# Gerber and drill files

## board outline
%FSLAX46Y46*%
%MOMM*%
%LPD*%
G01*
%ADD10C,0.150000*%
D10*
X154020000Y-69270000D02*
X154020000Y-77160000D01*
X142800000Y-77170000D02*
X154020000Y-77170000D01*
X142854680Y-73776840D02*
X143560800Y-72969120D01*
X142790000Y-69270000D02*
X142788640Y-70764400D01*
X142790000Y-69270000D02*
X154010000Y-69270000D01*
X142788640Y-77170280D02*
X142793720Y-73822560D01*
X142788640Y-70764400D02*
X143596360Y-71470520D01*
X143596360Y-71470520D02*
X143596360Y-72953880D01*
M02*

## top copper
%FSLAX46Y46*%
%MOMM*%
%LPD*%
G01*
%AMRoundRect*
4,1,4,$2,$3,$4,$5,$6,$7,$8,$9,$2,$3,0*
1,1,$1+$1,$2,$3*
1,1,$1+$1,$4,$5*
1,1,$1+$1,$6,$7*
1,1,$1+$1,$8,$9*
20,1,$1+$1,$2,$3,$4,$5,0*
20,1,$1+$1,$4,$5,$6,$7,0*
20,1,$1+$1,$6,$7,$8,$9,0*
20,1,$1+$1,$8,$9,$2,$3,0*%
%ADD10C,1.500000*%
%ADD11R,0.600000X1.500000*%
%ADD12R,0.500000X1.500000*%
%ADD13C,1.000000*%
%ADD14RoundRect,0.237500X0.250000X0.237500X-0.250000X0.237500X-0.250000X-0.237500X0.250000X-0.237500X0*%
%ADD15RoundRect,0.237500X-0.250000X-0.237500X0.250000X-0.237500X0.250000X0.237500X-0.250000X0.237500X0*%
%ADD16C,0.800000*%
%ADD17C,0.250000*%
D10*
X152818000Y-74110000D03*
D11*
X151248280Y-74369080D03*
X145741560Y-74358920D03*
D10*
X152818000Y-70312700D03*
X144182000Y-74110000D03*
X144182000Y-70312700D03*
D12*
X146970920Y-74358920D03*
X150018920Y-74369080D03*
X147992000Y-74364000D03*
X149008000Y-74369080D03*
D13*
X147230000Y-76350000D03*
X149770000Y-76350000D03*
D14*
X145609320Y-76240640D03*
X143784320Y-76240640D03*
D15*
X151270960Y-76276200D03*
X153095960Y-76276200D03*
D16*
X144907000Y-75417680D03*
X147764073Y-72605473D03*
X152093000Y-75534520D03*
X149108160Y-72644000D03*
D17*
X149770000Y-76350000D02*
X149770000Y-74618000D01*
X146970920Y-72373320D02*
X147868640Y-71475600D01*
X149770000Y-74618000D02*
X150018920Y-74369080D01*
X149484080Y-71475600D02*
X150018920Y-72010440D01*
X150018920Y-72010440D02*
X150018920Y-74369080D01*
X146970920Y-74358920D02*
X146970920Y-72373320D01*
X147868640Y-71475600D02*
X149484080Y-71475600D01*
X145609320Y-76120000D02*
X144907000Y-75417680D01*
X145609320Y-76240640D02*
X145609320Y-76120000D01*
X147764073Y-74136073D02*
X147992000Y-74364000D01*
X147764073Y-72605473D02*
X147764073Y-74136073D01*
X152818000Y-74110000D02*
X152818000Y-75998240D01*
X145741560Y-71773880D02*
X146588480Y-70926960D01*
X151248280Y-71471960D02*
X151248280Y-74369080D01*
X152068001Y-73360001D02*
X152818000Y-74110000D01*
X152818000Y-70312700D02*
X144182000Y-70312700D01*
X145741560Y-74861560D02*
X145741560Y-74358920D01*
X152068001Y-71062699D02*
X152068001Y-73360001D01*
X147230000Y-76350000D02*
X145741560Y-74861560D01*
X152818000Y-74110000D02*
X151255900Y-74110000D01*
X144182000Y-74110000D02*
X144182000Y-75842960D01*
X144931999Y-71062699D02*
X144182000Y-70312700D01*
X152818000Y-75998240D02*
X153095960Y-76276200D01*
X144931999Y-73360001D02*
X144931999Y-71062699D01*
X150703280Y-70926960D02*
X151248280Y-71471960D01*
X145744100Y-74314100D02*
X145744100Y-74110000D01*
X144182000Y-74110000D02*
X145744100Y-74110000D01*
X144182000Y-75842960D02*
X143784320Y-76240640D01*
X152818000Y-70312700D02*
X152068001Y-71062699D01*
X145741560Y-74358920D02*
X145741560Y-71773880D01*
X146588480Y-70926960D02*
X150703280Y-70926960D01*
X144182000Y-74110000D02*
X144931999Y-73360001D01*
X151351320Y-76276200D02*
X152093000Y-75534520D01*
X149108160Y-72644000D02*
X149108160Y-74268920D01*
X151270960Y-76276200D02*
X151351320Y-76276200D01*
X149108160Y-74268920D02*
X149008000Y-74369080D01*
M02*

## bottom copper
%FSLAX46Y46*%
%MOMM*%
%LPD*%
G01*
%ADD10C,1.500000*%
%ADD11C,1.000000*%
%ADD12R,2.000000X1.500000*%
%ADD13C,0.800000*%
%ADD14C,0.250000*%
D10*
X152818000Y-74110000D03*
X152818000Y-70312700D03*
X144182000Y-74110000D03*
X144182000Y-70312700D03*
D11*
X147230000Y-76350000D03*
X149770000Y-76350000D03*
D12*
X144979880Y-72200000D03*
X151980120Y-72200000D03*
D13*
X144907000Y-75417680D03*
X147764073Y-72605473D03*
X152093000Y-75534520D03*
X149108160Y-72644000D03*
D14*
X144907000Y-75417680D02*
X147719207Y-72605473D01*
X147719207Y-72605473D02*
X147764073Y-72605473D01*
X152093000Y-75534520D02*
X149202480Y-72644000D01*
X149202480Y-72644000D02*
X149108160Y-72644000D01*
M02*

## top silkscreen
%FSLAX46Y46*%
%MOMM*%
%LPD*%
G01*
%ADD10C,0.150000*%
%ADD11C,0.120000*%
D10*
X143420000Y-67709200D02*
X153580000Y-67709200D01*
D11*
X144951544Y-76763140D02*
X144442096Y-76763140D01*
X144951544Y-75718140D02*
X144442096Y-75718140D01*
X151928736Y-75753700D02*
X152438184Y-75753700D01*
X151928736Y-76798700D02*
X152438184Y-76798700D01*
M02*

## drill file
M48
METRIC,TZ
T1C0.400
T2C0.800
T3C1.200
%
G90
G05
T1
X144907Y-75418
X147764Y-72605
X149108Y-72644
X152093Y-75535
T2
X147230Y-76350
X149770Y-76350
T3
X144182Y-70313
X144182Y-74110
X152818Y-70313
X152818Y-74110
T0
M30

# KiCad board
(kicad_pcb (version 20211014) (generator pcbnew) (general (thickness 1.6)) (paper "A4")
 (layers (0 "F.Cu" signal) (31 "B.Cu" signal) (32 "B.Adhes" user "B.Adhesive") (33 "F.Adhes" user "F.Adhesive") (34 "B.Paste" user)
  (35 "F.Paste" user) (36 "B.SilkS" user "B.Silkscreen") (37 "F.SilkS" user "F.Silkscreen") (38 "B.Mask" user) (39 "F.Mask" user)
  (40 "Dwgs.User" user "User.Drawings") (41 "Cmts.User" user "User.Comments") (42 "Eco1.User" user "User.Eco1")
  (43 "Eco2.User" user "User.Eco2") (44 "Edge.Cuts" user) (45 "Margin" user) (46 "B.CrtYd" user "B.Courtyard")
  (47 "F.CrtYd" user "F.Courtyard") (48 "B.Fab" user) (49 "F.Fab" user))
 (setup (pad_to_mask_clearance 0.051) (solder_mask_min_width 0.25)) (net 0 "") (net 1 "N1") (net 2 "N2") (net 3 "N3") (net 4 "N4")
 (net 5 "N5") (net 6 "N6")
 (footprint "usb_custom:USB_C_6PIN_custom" (layer "F.Cu") (at 148.5 74.11)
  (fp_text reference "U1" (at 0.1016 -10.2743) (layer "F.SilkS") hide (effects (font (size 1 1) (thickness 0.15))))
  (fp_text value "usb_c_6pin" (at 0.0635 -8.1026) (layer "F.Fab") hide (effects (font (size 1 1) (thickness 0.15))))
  (fp_line (start -5.08 -6.4008) (end 5.08 -6.4008) (layer "F.SilkS") (width 0.15))
  (pad "1" thru_hole circle locked (at 4.318 0) (size 1.5 1.5) (drill 1.2) (layers *.Cu *.Mask) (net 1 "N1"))
  (pad "1" smd rect locked (at 2.74828 0.25908) (size 0.6 1.5) (layers "F.Cu" "F.Paste" "F.Mask") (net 1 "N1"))
  (pad "1" smd rect locked (at -2.75844 0.24892) (size 0.6 1.5) (layers "F.Cu" "F.Paste" "F.Mask") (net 1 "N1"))
  (pad "1" thru_hole circle locked (at 4.318 -3.7973) (size 1.5 1.5) (drill 1.2) (layers *.Cu *.Mask) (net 1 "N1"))
  (pad "1" thru_hole circle locked (at -4.318 0) (size 1.5 1.5) (drill 1.2) (layers *.Cu *.Mask) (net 1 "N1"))
  (pad "1" thru_hole circle locked (at -4.318 -3.7973) (size 1.5 1.5) (drill 1.2) (layers *.Cu *.Mask) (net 1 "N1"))
  (pad "2" smd rect locked (at -1.52908 0.24892) (size 0.5 1.5) (layers "F.Cu" "F.Paste" "F.Mask") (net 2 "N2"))
  (pad "2" smd rect locked (at 1.51892 0.25908) (size 0.5 1.5) (layers "F.Cu" "F.Paste" "F.Mask") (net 2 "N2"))
  (pad "3" smd rect locked (at -0.508 0.254) (size 0.5 1.5) (layers "F.Cu" "F.Paste" "F.Mask") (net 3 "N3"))
  (pad "4" smd rect locked (at 0.508 0.25908) (size 0.5 1.5) (layers "F.Cu" "F.Paste" "F.Mask") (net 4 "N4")))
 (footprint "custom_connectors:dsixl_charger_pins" (layer "F.Cu") (at 148.5 76.35)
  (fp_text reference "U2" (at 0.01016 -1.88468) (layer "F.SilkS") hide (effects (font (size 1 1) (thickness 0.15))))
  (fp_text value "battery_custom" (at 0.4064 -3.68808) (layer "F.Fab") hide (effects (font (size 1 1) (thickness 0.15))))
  (pad "1" thru_hole circle locked (at -1.27 0) (size 1 1) (drill 0.8) (layers *.Cu *.Mask) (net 1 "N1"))
  (pad "2" thru_hole circle locked (at 1.27 0) (size 1 1) (drill 0.8) (layers *.Cu *.Mask) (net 2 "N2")))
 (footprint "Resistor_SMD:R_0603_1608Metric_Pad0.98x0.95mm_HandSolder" (layer "F.Cu") (at 144.69682 76.24064 180)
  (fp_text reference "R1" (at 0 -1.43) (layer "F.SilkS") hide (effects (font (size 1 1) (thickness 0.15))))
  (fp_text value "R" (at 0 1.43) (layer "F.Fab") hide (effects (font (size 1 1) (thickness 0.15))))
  (fp_line (start -0.254724 -0.5225) (end 0.254724 -0.5225) (layer "F.SilkS") (width 0.12))
  (fp_line (start -0.254724 0.5225) (end 0.254724 0.5225) (layer "F.SilkS") (width 0.12))
  (pad "1" smd roundrect locked (at -0.9125 0 180) (size 0.975 0.95) (layers "F.Cu" "F.Paste" "F.Mask") (roundrect_rratio 0.25) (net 3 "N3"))
  (pad "2" smd roundrect locked (at 0.9125 0 180) (size 0.975 0.95) (layers "F.Cu" "F.Paste" "F.Mask") (roundrect_rratio 0.25) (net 1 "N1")))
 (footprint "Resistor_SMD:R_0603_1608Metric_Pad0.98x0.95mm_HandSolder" (layer "F.Cu") (at 152.18346 76.2762)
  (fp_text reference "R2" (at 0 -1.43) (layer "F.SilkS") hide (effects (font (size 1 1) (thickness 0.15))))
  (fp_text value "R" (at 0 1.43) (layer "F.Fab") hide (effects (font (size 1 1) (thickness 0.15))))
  (fp_line (start -0.254724 -0.5225) (end 0.254724 -0.5225) (layer "F.SilkS") (width 0.12))
  (fp_line (start -0.254724 0.5225) (end 0.254724 0.5225) (layer "F.SilkS") (width 0.12))
  (pad "1" smd roundrect locked (at -0.9125 0) (size 0.975 0.95) (layers "F.Cu" "F.Paste" "F.Mask") (roundrect_rratio 0.25) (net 4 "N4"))
  (pad "2" smd roundrect locked (at 0.9125 0) (size 0.975 0.95) (layers "F.Cu" "F.Paste" "F.Mask") (roundrect_rratio 0.25) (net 1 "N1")))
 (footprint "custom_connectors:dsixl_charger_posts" (layer "B.Cu") (at 148.48 72.2)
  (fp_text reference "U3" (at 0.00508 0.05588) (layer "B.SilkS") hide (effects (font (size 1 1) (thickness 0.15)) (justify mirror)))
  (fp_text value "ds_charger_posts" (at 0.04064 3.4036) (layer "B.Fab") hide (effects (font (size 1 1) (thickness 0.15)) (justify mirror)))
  (pad "1" smd rect locked (at -3.50012 0) (size 2 1.5) (layers "B.Cu" "B.Paste" "B.Mask") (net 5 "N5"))
  (pad "2" smd rect locked (at 3.50012 0) (size 2 1.5) (layers "B.Cu" "B.Paste" "B.Mask") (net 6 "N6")))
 (gr_line (start 154.02 69.27) (end 154.02 77.16) (layer "Edge.Cuts") (width 0.15))
 (gr_line (start 142.8 77.17) (end 154.02 77.17) (layer "Edge.Cuts") (width 0.15))
 (gr_line (start 142.85468 73.77684) (end 143.5608 72.96912) (layer "Edge.Cuts") (width 0.15))
 (gr_line (start 142.79 69.27) (end 142.78864 70.7644) (layer "Edge.Cuts") (width 0.15))
 (gr_line (start 142.79 69.27) (end 154.01 69.27) (layer "Edge.Cuts") (width 0.15))
 (gr_line (start 142.78864 77.17028) (end 142.79372 73.82256) (layer "Edge.Cuts") (width 0.15))
 (gr_line (start 142.78864 70.7644) (end 143.59636 71.47052) (layer "Edge.Cuts") (width 0.15))
 (gr_line (start 143.59636 71.47052) (end 143.59636 72.95388) (layer "Edge.Cuts") (width 0.15))
 (segment (start 149.77 76.35) (end 149.77 74.618) (width 0.25) (layer "F.Cu") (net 2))
 (segment (start 146.97092 72.37332) (end 147.86864 71.4756) (width 0.25) (layer "F.Cu") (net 2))
 (segment (start 149.77 74.618) (end 150.01892 74.36908) (width 0.25) (layer "F.Cu") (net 2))
 (segment (start 149.48408 71.4756) (end 150.01892 72.01044) (width 0.25) (layer "F.Cu") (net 2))
 (segment (start 150.01892 72.01044) (end 150.01892 74.36908) (width 0.25) (layer "F.Cu") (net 2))
 (segment (start 146.97092 74.35892) (end 146.97092 72.37332) (width 0.25) (layer "F.Cu") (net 2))
 (segment (start 147.86864 71.4756) (end 149.48408 71.4756) (width 0.25) (layer "F.Cu") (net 2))
 (segment (start 145.60932 76.12) (end 144.907 75.41768) (width 0.25) (layer "F.Cu") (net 3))
 (segment (start 145.60932 76.24064) (end 145.60932 76.12) (width 0.25) (layer "F.Cu") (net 3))
 (segment (start 147.764073 74.136073) (end 147.992 74.364) (width 0.25) (layer "F.Cu") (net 3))
 (segment (start 147.764073 72.605473) (end 147.764073 74.136073) (width 0.25) (layer "F.Cu") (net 3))
 (via (at 144.907 75.41768) (size 0.8) (drill 0.4) (layers "F.Cu" "B.Cu") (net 3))
 (via (at 147.764073 72.605473) (size 0.8) (drill 0.4) (layers "F.Cu" "B.Cu") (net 3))
 (segment (start 144.907 75.41768) (end 147.719207 72.605473) (width 0.25) (layer "B.Cu") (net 3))
 (segment (start 147.719207 72.605473) (end 147.764073 72.605473) (width 0.25) (layer "B.Cu") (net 3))
 (segment (start 152.818 74.11) (end 152.818 75.99824) (width 0.25) (layer "F.Cu") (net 1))
 (segment (start 145.74156 71.77388) (end 146.58848 70.92696) (width 0.25) (layer "F.Cu") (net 1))
 (segment (start 151.24828 71.47196) (end 151.24828 74.36908) (width 0.25) (layer "F.Cu") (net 1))
 (segment (start 152.068001 73.360001) (end 152.818 74.11) (width 0.25) (layer "F.Cu") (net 1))
 (segment (start 152.818 70.3127) (end 144.182 70.3127) (width 0.25) (layer "F.Cu") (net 1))
 (segment (start 145.74156 74.86156) (end 145.74156 74.35892) (width 0.25) (layer "F.Cu") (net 1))
 (segment (start 152.068001 71.062699) (end 152.068001 73.360001) (width 0.25) (layer "F.Cu") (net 1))
 (segment (start 147.23 76.35) (end 145.74156 74.86156) (width 0.25) (layer "F.Cu") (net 1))
 (segment (start 152.818 74.11) (end 151.2559 74.11) (width 0.25) (layer "F.Cu") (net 1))
 (segment (start 144.182 74.11) (end 144.182 75.84296) (width 0.25) (layer "F.Cu") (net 1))
 (segment (start 144.931999 71.062699) (end 144.182 70.3127) (width 0.25) (layer "F.Cu") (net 1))
 (segment (start 152.818 75.99824) (end 153.09596 76.2762) (width 0.25) (layer "F.Cu") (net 1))
 (segment (start 144.931999 73.360001) (end 144.931999 71.062699) (width 0.25) (layer "F.Cu") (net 1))
 (segment (start 150.70328 70.92696) (end 151.24828 71.47196) (width 0.25) (layer "F.Cu") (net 1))
 (segment (start 145.7441 74.3141) (end 145.7441 74.11) (width 0.25) (layer "F.Cu") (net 1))
 (segment (start 144.182 74.11) (end 145.7441 74.11) (width 0.25) (layer "F.Cu") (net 1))
 (segment (start 144.182 75.84296) (end 143.78432 76.24064) (width 0.25) (layer "F.Cu") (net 1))
 (segment (start 152.818 70.3127) (end 152.068001 71.062699) (width 0.25) (layer "F.Cu") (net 1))
 (segment (start 145.74156 74.35892) (end 145.74156 71.77388) (width 0.25) (layer "F.Cu") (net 1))
 (segment (start 146.58848 70.92696) (end 150.70328 70.92696) (width 0.25) (layer "F.Cu") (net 1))
 (segment (start 144.182 74.11) (end 144.931999 73.360001) (width 0.25) (layer "F.Cu") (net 1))
 (segment (start 151.35132 76.2762) (end 152.093 75.53452) (width 0.25) (layer "F.Cu") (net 4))
 (segment (start 149.10816 72.644) (end 149.10816 74.26892) (width 0.25) (layer "F.Cu") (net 4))
 (segment (start 151.27096 76.2762) (end 151.35132 76.2762) (width 0.25) (layer "F.Cu") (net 4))
 (segment (start 149.10816 74.26892) (end 149.008 74.36908) (width 0.25) (layer "F.Cu") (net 4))
 (via (at 152.093 75.53452) (size 0.8) (drill 0.4) (layers "F.Cu" "B.Cu") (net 4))
 (via (at 149.10816 72.644) (size 0.8) (drill 0.4) (layers "F.Cu" "B.Cu") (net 4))
 (segment (start 152.093 75.53452) (end 149.20248 72.644) (width 0.25) (layer "B.Cu") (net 4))
 (segment (start 149.20248 72.644) (end 149.10816 72.644) (width 0.25) (layer "B.Cu") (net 4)))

